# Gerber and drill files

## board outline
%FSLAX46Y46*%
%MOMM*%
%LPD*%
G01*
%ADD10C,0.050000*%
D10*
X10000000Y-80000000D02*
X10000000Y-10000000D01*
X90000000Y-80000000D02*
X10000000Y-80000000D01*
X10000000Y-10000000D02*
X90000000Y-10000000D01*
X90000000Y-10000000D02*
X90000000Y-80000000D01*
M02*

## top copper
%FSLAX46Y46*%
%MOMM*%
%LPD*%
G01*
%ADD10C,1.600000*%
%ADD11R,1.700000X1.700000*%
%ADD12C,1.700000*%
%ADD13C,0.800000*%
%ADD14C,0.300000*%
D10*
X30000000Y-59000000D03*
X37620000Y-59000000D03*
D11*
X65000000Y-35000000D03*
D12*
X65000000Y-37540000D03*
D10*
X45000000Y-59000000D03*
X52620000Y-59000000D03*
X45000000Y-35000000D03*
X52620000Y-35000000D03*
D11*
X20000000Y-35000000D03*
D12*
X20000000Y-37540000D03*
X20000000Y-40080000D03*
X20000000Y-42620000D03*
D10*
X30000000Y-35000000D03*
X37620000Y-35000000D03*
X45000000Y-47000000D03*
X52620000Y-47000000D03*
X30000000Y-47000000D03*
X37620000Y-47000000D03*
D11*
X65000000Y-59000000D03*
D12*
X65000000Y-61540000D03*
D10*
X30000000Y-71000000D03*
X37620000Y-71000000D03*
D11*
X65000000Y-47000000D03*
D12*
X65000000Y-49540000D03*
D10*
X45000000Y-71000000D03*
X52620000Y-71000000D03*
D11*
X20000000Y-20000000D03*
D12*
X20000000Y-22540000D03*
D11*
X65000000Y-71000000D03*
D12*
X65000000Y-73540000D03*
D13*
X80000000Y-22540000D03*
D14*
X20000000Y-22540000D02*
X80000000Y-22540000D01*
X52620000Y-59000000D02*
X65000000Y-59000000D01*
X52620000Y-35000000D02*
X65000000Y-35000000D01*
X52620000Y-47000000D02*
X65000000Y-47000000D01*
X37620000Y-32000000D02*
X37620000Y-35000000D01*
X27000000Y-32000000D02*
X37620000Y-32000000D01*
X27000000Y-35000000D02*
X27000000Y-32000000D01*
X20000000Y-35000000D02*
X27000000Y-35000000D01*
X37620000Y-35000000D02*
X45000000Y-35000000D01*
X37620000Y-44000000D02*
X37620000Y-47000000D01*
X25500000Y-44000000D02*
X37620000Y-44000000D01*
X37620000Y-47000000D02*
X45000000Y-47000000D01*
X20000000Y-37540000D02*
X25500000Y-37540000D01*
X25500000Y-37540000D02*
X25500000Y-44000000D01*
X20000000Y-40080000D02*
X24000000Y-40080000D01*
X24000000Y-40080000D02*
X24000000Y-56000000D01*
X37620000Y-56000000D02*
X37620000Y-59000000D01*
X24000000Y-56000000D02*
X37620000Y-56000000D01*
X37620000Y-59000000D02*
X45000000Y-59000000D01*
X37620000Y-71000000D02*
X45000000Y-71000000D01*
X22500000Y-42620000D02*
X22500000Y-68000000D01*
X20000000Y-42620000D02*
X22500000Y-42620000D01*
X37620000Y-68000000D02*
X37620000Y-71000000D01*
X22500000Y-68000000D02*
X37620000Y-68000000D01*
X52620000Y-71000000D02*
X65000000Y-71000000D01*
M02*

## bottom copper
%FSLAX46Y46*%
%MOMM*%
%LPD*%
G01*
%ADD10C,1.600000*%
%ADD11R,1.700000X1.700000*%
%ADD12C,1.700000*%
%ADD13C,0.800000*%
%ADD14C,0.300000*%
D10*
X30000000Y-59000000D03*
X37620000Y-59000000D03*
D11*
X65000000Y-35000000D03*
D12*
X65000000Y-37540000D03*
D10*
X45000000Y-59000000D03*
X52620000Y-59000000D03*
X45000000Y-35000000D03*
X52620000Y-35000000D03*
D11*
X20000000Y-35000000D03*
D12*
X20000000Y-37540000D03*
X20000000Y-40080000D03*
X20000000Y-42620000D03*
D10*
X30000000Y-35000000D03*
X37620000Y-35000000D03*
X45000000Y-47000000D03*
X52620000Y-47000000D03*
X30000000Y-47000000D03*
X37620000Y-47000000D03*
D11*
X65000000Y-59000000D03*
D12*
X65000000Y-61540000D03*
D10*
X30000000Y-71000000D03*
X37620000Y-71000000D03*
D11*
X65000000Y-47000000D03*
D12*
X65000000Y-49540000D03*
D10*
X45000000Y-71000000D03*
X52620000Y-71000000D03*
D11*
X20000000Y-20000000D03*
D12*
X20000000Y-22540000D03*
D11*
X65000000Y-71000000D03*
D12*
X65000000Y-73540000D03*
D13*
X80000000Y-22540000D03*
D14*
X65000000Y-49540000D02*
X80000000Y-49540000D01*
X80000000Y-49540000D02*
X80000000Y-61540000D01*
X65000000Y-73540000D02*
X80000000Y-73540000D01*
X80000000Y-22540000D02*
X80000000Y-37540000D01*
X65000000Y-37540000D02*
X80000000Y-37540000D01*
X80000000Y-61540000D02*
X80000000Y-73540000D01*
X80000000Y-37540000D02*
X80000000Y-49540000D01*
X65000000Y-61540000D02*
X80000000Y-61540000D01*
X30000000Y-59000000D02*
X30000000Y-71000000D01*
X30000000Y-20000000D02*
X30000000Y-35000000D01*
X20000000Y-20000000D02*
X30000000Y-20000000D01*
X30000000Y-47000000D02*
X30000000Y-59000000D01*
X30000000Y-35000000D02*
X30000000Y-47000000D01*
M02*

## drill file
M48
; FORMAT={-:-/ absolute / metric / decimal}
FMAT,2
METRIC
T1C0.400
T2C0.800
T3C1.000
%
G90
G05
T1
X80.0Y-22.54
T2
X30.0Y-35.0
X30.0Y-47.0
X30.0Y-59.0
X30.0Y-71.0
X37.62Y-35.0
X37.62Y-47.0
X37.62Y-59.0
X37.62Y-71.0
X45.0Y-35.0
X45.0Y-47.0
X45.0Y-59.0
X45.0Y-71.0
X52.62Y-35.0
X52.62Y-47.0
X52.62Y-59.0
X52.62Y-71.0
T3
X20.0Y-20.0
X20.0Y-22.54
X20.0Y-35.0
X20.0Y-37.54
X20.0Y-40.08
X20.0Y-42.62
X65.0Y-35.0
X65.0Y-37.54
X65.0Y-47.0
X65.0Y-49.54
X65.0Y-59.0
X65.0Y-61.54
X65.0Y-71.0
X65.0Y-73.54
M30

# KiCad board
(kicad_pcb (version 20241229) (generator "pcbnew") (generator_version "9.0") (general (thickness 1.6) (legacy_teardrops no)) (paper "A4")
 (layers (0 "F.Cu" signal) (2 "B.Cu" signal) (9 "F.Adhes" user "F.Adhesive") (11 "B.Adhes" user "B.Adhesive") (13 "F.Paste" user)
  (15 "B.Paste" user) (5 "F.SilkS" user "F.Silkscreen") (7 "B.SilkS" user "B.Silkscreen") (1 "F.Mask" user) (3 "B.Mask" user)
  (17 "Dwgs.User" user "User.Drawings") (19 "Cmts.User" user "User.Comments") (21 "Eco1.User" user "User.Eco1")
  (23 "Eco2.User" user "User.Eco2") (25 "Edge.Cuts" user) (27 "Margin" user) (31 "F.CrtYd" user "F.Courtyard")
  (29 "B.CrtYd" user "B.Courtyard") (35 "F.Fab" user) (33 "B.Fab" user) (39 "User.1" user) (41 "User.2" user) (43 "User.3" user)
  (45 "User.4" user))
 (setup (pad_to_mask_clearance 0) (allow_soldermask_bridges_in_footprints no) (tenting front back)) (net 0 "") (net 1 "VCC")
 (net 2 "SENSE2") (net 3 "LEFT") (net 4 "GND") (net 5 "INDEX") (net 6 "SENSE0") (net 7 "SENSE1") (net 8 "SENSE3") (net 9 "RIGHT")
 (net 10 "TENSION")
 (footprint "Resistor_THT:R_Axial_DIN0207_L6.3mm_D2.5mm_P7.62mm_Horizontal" (layer "F.Cu") (at 30 59)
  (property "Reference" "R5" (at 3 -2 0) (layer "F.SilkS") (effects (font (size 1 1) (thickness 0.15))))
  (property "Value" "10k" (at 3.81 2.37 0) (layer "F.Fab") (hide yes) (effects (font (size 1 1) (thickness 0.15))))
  (pad "1" thru_hole circle (at 0 0) (size 1.6 1.6) (drill 0.8) (layers "*.Cu" "*.Mask") (remove_unused_layers no) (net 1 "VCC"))
  (pad "2" thru_hole circle (at 7.62 0) (size 1.6 1.6) (drill 0.8) (layers "*.Cu" "*.Mask") (remove_unused_layers no) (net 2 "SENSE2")))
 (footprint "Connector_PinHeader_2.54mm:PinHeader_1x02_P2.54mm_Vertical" (layer "F.Cu") (at 65 35)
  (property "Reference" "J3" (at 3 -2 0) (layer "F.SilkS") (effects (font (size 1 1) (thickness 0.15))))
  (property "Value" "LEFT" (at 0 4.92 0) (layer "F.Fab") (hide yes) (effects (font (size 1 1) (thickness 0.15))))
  (pad "1" thru_hole rect (at 0 0) (size 1.7 1.7) (drill 1) (layers "*.Cu" "*.Mask") (remove_unused_layers no) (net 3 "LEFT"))
  (pad "2" thru_hole circle (at 0 2.54) (size 1.7 1.7) (drill 1) (layers "*.Cu" "*.Mask") (remove_unused_layers no) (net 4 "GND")))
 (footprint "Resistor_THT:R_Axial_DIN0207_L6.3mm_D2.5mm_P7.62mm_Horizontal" (layer "F.Cu") (at 45 59)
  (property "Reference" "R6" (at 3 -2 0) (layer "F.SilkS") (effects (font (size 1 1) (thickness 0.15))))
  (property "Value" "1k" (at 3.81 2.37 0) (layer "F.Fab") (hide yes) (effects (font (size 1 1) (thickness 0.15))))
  (pad "1" thru_hole circle (at 0 0) (size 1.6 1.6) (drill 0.8) (layers "*.Cu" "*.Mask") (remove_unused_layers no) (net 2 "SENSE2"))
  (pad "2" thru_hole circle (at 7.62 0) (size 1.6 1.6) (drill 0.8) (layers "*.Cu" "*.Mask") (remove_unused_layers no) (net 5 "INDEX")))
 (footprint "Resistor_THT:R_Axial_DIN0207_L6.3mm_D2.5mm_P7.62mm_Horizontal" (layer "F.Cu") (at 45 35)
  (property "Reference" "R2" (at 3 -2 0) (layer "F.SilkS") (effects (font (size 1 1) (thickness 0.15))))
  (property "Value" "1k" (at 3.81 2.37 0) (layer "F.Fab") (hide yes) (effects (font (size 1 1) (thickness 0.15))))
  (pad "1" thru_hole circle (at 0 0) (size 1.6 1.6) (drill 0.8) (layers "*.Cu" "*.Mask") (remove_unused_layers no) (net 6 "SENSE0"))
  (pad "2" thru_hole circle (at 7.62 0) (size 1.6 1.6) (drill 0.8) (layers "*.Cu" "*.Mask") (remove_unused_layers no) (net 3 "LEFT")))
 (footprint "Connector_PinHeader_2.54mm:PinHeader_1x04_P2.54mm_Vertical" (layer "F.Cu") (at 20 35)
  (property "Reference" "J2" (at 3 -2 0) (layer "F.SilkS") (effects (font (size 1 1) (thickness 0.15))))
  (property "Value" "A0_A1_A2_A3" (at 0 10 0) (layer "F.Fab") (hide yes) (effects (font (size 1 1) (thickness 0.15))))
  (pad "1" thru_hole rect (at 0 0) (size 1.7 1.7) (drill 1) (layers "*.Cu" "*.Mask") (remove_unused_layers no) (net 6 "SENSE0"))
  (pad "2" thru_hole circle (at 0 2.54) (size 1.7 1.7) (drill 1) (layers "*.Cu" "*.Mask") (remove_unused_layers no) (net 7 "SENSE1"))
  (pad "3" thru_hole circle (at 0 5.08) (size 1.7 1.7) (drill 1) (layers "*.Cu" "*.Mask") (remove_unused_layers no) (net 2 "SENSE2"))
  (pad "4" thru_hole circle (at 0 7.62) (size 1.7 1.7) (drill 1) (layers "*.Cu" "*.Mask") (remove_unused_layers no) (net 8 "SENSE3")))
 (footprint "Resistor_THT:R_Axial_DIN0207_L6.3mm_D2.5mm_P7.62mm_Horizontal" (layer "F.Cu") (at 30 35)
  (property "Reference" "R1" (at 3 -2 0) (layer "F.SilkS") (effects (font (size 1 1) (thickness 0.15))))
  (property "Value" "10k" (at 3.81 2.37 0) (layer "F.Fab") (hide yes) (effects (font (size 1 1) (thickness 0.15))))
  (pad "1" thru_hole circle (at 0 0) (size 1.6 1.6) (drill 0.8) (layers "*.Cu" "*.Mask") (remove_unused_layers no) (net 1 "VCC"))
  (pad "2" thru_hole circle (at 7.62 0) (size 1.6 1.6) (drill 0.8) (layers "*.Cu" "*.Mask") (remove_unused_layers no) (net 6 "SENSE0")))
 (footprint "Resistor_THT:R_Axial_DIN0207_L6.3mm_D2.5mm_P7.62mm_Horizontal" (layer "F.Cu") (at 45 47)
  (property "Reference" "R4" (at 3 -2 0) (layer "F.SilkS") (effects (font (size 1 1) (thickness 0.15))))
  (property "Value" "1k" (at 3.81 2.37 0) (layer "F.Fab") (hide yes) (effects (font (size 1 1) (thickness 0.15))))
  (pad "1" thru_hole circle (at 0 0) (size 1.6 1.6) (drill 0.8) (layers "*.Cu" "*.Mask") (remove_unused_layers no) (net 7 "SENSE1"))
  (pad "2" thru_hole circle (at 7.62 0) (size 1.6 1.6) (drill 0.8) (layers "*.Cu" "*.Mask") (remove_unused_layers no) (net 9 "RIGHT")))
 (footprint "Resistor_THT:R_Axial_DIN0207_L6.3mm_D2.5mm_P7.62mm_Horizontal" (layer "F.Cu") (at 30 47)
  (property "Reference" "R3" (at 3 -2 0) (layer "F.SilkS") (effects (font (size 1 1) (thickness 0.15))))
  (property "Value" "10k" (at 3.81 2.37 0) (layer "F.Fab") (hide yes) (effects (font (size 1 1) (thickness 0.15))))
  (pad "1" thru_hole circle (at 0 0) (size 1.6 1.6) (drill 0.8) (layers "*.Cu" "*.Mask") (remove_unused_layers no) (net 1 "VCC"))
  (pad "2" thru_hole circle (at 7.62 0) (size 1.6 1.6) (drill 0.8) (layers "*.Cu" "*.Mask") (remove_unused_layers no) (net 7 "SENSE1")))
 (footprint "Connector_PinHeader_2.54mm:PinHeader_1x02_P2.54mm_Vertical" (layer "F.Cu") (at 65 59)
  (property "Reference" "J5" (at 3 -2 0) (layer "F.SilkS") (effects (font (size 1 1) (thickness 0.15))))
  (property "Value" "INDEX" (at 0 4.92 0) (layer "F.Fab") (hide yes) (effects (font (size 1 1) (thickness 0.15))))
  (pad "1" thru_hole rect (at 0 0) (size 1.7 1.7) (drill 1) (layers "*.Cu" "*.Mask") (remove_unused_layers no) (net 5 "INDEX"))
  (pad "2" thru_hole circle (at 0 2.54) (size 1.7 1.7) (drill 1) (layers "*.Cu" "*.Mask") (remove_unused_layers no) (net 4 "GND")))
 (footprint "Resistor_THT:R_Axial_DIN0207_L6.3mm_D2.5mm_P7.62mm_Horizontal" (layer "F.Cu") (at 30 71)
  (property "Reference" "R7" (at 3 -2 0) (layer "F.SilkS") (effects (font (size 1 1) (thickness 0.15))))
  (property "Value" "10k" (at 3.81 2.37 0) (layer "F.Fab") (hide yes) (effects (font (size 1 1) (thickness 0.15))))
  (pad "1" thru_hole circle (at 0 0) (size 1.6 1.6) (drill 0.8) (layers "*.Cu" "*.Mask") (remove_unused_layers no) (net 1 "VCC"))
  (pad "2" thru_hole circle (at 7.62 0) (size 1.6 1.6) (drill 0.8) (layers "*.Cu" "*.Mask") (remove_unused_layers no) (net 8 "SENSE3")))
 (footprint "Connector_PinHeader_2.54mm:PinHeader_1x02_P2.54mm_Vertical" (layer "F.Cu") (at 65 47)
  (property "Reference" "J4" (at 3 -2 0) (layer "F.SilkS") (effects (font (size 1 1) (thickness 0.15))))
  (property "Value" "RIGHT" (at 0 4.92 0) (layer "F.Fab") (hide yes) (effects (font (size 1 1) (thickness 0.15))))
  (pad "1" thru_hole rect (at 0 0) (size 1.7 1.7) (drill 1) (layers "*.Cu" "*.Mask") (remove_unused_layers no) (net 9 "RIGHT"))
  (pad "2" thru_hole circle (at 0 2.54) (size 1.7 1.7) (drill 1) (layers "*.Cu" "*.Mask") (remove_unused_layers no) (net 4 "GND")))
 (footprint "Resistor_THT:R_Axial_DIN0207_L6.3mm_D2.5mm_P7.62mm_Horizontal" (layer "F.Cu") (at 45 71)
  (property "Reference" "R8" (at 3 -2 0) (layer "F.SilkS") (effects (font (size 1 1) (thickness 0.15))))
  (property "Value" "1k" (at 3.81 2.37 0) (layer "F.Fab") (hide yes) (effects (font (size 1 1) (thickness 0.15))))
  (pad "1" thru_hole circle (at 0 0) (size 1.6 1.6) (drill 0.8) (layers "*.Cu" "*.Mask") (remove_unused_layers no) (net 8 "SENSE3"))
  (pad "2" thru_hole circle (at 7.62 0) (size 1.6 1.6) (drill 0.8) (layers "*.Cu" "*.Mask") (remove_unused_layers no) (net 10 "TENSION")))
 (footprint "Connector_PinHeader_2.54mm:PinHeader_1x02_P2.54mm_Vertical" (layer "F.Cu") (at 20 20)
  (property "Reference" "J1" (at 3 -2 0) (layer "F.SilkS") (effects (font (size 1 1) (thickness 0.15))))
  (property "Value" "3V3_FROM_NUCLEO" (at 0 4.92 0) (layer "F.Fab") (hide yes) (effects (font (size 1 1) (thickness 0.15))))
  (pad "1" thru_hole rect (at 0 0) (size 1.7 1.7) (drill 1) (layers "*.Cu" "*.Mask") (remove_unused_layers no) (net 1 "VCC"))
  (pad "2" thru_hole circle (at 0 2.54) (size 1.7 1.7) (drill 1) (layers "*.Cu" "*.Mask") (remove_unused_layers no) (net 4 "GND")))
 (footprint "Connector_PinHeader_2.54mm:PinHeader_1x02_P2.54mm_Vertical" (layer "F.Cu") (at 65 71)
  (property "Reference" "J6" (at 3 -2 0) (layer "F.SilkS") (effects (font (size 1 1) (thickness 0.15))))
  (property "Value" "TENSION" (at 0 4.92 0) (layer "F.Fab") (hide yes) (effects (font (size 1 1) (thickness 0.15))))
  (pad "1" thru_hole rect (at 0 0) (size 1.7 1.7) (drill 1) (layers "*.Cu" "*.Mask") (remove_unused_layers no) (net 10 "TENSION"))
  (pad "2" thru_hole circle (at 0 2.54) (size 1.7 1.7) (drill 1) (layers "*.Cu" "*.Mask") (remove_unused_layers no) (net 4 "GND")))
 (gr_line (start 10 80) (end 10 10) (stroke (width 0.05) (type default)) (layer "Edge.Cuts"))
 (gr_line (start 90 80) (end 10 80) (stroke (width 0.05) (type default)) (layer "Edge.Cuts"))
 (gr_line (start 10 10) (end 90 10) (stroke (width 0.05) (type default)) (layer "Edge.Cuts"))
 (gr_line (start 90 10) (end 90 80) (stroke (width 0.05) (type default)) (layer "Edge.Cuts"))
 (segment (start 20 22.54) (end 80 22.54) (width 0.3) (layer "F.Cu") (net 4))
 (via (at 80 22.54) (size 0.8) (drill 0.4) (layers "F.Cu" "B.Cu") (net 4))
 (segment (start 65 49.54) (end 80 49.54) (width 0.3) (layer "B.Cu") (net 4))
 (segment (start 80 49.54) (end 80 61.54) (width 0.3) (layer "B.Cu") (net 4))
 (segment (start 65 73.54) (end 80 73.54) (width 0.3) (layer "B.Cu") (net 4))
 (segment (start 80 22.54) (end 80 37.54) (width 0.3) (layer "B.Cu") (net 4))
 (segment (start 65 37.54) (end 80 37.54) (width 0.3) (layer "B.Cu") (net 4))
 (segment (start 80 61.54) (end 80 73.54) (width 0.3) (layer "B.Cu") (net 4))
 (segment (start 80 37.54) (end 80 49.54) (width 0.3) (layer "B.Cu") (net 4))
 (segment (start 65 61.54) (end 80 61.54) (width 0.3) (layer "B.Cu") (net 4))
 (segment (start 52.62 59) (end 65 59) (width 0.3) (layer "F.Cu") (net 5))
 (segment (start 52.62 35) (end 65 35) (width 0.3) (layer "F.Cu") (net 3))
 (segment (start 52.62 47) (end 65 47) (width 0.3) (layer "F.Cu") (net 9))
 (segment (start 37.62 32) (end 37.62 35) (width 0.3) (layer "F.Cu") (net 6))
 (segment (start 27 32) (end 37.62 32) (width 0.3) (layer "F.Cu") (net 6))
 (segment (start 27 35) (end 27 32) (width 0.3) (layer "F.Cu") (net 6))
 (segment (start 20 35) (end 27 35) (width 0.3) (layer "F.Cu") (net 6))
 (segment (start 37.62 35) (end 45 35) (width 0.3) (layer "F.Cu") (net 6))
 (segment (start 37.62 44) (end 37.62 47) (width 0.3) (layer "F.Cu") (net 7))
 (segment (start 25.5 44) (end 37.62 44) (width 0.3) (layer "F.Cu") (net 7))
 (segment (start 37.62 47) (end 45 47) (width 0.3) (layer "F.Cu") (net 7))
 (segment (start 20 37.54) (end 25.5 37.54) (width 0.3) (layer "F.Cu") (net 7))
 (segment (start 25.5 37.54) (end 25.5 44) (width 0.3) (layer "F.Cu") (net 7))
 (segment (start 20 40.08) (end 24 40.08) (width 0.3) (layer "F.Cu") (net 2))
 (segment (start 24 40.08) (end 24 56) (width 0.3) (layer "F.Cu") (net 2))
 (segment (start 37.62 56) (end 37.62 59) (width 0.3) (layer "F.Cu") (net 2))
 (segment (start 24 56) (end 37.62 56) (width 0.3) (layer "F.Cu") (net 2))
 (segment (start 37.62 59) (end 45 59) (width 0.3) (layer "F.Cu") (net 2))
 (segment (start 37.62 71) (end 45 71) (width 0.3) (layer "F.Cu") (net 8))
 (segment (start 22.5 42.62) (end 22.5 68) (width 0.3) (layer "F.Cu") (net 8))
 (segment (start 20 42.62) (end 22.5 42.62) (width 0.3) (layer "F.Cu") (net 8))
 (segment (start 37.62 68) (end 37.62 71) (width 0.3) (layer "F.Cu") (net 8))
 (segment (start 22.5 68) (end 37.62 68) (width 0.3) (layer "F.Cu") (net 8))
 (segment (start 52.62 71) (end 65 71) (width 0.3) (layer "F.Cu") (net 10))
 (segment (start 30 59) (end 30 71) (width 0.3) (layer "B.Cu") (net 1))
 (segment (start 30 20) (end 30 35) (width 0.3) (layer "B.Cu") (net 1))
 (segment (start 20 20) (end 30 20) (width 0.3) (layer "B.Cu") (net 1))
 (segment (start 30 47) (end 30 59) (width 0.3) (layer "B.Cu") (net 1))
 (segment (start 30 35) (end 30 47) (width 0.3) (layer "B.Cu") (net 1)))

